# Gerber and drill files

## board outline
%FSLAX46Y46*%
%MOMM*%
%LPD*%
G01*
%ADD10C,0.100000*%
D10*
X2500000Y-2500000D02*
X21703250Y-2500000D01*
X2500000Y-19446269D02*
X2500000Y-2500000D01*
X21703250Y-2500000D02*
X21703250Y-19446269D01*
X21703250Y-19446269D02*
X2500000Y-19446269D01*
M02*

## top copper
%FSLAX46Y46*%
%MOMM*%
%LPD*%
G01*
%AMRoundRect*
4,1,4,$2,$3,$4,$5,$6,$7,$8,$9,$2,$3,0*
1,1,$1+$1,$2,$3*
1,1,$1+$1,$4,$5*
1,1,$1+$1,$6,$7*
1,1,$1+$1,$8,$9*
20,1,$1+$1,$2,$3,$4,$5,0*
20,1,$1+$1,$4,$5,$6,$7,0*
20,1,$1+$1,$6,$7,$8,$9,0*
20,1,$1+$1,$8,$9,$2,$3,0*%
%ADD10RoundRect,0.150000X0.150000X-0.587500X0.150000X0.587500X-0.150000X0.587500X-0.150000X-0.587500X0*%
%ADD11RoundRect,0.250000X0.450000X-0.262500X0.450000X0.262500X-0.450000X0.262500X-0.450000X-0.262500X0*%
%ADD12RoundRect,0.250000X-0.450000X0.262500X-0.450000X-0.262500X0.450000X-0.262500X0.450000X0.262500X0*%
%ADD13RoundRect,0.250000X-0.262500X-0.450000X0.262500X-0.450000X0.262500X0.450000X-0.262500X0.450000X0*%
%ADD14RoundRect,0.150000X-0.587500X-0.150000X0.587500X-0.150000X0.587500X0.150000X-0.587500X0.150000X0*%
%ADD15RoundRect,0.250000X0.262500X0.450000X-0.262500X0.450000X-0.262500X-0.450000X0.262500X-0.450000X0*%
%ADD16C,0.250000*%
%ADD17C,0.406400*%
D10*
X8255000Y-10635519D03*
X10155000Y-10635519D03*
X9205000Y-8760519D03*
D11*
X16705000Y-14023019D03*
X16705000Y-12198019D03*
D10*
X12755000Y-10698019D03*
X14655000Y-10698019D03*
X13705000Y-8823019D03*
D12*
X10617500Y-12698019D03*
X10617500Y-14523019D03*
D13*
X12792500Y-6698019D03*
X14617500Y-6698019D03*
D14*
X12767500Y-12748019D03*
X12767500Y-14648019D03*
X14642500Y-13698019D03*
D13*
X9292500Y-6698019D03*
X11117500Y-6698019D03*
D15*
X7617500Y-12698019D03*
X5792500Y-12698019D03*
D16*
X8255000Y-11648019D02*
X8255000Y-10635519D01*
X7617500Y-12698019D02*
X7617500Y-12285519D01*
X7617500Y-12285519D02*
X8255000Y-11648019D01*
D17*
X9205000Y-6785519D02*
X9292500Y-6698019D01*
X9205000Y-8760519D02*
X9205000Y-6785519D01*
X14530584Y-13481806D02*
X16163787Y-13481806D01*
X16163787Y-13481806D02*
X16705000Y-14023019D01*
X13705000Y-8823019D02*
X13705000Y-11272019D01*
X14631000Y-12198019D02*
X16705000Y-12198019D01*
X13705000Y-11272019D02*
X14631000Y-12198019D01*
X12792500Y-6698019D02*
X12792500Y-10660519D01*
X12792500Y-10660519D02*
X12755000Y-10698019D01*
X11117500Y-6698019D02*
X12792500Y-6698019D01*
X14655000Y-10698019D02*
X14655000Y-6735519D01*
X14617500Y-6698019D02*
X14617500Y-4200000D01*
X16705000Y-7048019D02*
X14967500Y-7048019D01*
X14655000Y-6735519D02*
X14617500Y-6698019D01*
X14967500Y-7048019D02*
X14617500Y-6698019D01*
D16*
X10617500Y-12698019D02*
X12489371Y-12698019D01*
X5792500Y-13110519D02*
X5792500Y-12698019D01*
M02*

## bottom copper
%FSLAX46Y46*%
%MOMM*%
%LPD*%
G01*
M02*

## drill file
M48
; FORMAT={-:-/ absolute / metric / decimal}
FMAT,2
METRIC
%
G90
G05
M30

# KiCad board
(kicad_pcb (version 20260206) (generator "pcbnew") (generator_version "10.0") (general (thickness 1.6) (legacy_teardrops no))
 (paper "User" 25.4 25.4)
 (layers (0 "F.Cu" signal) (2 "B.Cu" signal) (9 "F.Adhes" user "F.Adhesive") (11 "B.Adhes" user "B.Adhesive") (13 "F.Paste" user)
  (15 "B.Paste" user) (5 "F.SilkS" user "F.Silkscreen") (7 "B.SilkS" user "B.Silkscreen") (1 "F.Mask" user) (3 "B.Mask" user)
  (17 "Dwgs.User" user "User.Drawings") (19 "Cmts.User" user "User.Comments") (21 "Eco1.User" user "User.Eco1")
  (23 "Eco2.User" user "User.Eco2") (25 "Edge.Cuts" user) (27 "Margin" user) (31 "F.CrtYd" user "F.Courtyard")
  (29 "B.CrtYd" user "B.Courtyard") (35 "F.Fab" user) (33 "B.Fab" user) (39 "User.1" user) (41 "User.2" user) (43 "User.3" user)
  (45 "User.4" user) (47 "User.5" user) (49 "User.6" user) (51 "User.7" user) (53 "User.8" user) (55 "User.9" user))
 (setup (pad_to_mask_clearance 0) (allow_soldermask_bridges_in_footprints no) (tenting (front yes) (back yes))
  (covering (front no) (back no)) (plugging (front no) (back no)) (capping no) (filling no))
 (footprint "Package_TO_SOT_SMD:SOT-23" (layer "F.Cu") (at 9.205 9.698019 90)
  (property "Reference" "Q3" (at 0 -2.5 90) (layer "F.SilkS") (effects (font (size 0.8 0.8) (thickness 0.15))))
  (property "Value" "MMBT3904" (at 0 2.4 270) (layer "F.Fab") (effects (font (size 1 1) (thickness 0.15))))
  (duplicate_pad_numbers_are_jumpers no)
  (pad "1" smd roundrect (at -0.9375 -0.95 90) (size 1.475 0.6) (layers "F.Cu" "F.Mask" "F.Paste") (roundrect_rratio 0.25)
   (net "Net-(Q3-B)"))
  (pad "2" smd roundrect (at -0.9375 0.95 90) (size 1.475 0.6) (layers "F.Cu" "F.Mask" "F.Paste") (roundrect_rratio 0.25) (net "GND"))
  (pad "3" smd roundrect (at 0.9375 0 90) (size 1.475 0.6) (layers "F.Cu" "F.Mask" "F.Paste") (roundrect_rratio 0.25) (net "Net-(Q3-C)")))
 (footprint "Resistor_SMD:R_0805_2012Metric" (layer "F.Cu") (at 16.705 13.110519 90)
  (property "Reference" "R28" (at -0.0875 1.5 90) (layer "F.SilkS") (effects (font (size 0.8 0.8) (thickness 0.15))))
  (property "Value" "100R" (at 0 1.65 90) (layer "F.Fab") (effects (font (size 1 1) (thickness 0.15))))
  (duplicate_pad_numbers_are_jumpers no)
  (pad "1" smd roundrect (at -0.9125 0 90) (size 1.025 1.4) (layers "F.Cu" "F.Mask" "F.Paste") (roundrect_rratio 0.243902439)
   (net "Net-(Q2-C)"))
  (pad "2" smd roundrect (at 0.9125 0 90) (size 1.025 1.4) (layers "F.Cu" "F.Mask" "F.Paste") (roundrect_rratio 0.243902439) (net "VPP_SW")))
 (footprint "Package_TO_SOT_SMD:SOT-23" (layer "F.Cu") (at 13.705 9.760519 90)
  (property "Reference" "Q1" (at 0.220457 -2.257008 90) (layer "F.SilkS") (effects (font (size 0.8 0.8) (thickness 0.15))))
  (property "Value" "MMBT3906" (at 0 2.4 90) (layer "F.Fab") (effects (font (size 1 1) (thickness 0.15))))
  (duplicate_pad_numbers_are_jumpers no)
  (pad "1" smd roundrect (at -0.9375 -0.95 90) (size 1.475 0.6) (layers "F.Cu" "F.Mask" "F.Paste") (roundrect_rratio 0.25)
   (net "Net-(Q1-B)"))
  (pad "2" smd roundrect (at -0.9375 0.95 90) (size 1.475 0.6) (layers "F.Cu" "F.Mask" "F.Paste") (roundrect_rratio 0.25) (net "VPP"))
  (pad "3" smd roundrect (at 0.9375 0 90) (size 1.475 0.6) (layers "F.Cu" "F.Mask" "F.Paste") (roundrect_rratio 0.25) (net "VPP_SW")))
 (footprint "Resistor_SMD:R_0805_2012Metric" (layer "F.Cu") (at 10.6175 13.610519 -90)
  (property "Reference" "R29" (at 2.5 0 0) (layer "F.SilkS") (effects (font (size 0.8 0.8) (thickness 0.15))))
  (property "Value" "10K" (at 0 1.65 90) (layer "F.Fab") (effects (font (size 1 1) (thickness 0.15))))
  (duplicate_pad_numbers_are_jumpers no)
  (pad "1" smd roundrect (at -0.9125 0 270) (size 1.025 1.4) (layers "F.Cu" "F.Mask" "F.Paste") (roundrect_rratio 0.243902439)
   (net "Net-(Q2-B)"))
  (pad "2" smd roundrect (at 0.9125 0 270) (size 1.025 1.4) (layers "F.Cu" "F.Mask" "F.Paste") (roundrect_rratio 0.243902439)
   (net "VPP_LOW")))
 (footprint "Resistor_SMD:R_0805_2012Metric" (layer "F.Cu") (at 13.705 6.698019)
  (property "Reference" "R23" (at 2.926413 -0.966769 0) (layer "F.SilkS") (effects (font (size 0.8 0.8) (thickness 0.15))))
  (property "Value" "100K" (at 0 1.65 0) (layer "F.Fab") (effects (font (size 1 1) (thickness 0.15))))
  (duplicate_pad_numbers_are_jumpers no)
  (pad "1" smd roundrect (at -0.9125 0) (size 1.025 1.4) (layers "F.Cu" "F.Mask" "F.Paste") (roundrect_rratio 0.243902439)
   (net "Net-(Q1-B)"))
  (pad "2" smd roundrect (at 0.9125 0) (size 1.025 1.4) (layers "F.Cu" "F.Mask" "F.Paste") (roundrect_rratio 0.243902439) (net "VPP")))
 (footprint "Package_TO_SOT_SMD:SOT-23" (layer "F.Cu") (at 13.705 13.698019)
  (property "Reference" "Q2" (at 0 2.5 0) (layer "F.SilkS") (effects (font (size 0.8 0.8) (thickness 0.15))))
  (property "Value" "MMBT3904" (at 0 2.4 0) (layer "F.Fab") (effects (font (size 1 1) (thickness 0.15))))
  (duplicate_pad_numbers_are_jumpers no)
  (pad "1" smd roundrect (at -0.9375 -0.95) (size 1.475 0.6) (layers "F.Cu" "F.Mask" "F.Paste") (roundrect_rratio 0.25) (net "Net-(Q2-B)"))
  (pad "2" smd roundrect (at -0.9375 0.95) (size 1.475 0.6) (layers "F.Cu" "F.Mask" "F.Paste") (roundrect_rratio 0.25) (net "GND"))
  (pad "3" smd roundrect (at 0.9375 0) (size 1.475 0.6) (layers "F.Cu" "F.Mask" "F.Paste") (roundrect_rratio 0.25) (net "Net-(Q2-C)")))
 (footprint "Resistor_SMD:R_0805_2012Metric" (layer "F.Cu") (at 10.205 6.698019)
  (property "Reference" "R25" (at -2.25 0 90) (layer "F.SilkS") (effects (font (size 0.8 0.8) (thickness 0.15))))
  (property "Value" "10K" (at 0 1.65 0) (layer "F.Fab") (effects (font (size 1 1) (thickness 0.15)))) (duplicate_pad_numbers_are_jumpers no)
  (pad "1" smd roundrect (at -0.9125 0) (size 1.025 1.4) (layers "F.Cu" "F.Mask" "F.Paste") (roundrect_rratio 0.243902439)
   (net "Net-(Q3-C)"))
  (pad "2" smd roundrect (at 0.9125 0) (size 1.025 1.4) (layers "F.Cu" "F.Mask" "F.Paste") (roundrect_rratio 0.243902439) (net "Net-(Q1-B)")))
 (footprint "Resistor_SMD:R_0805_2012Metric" (layer "F.Cu") (at 6.705 12.698019 180)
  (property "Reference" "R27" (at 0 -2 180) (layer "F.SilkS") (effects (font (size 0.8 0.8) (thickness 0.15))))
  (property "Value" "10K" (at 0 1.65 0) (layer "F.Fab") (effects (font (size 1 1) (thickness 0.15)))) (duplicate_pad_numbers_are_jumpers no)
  (pad "1" smd roundrect (at -0.9125 0 180) (size 1.025 1.4) (layers "F.Cu" "F.Mask" "F.Paste") (roundrect_rratio 0.243902439)
   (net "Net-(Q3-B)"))
  (pad "2" smd roundrect (at 0.9125 0 180) (size 1.025 1.4) (layers "F.Cu" "F.Mask" "F.Paste") (roundrect_rratio 0.243902439)
   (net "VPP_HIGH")))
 (gr_line (start 2.5 2.5) (end 21.70325 2.5) (stroke (width 0.1) (type default)) (layer "Edge.Cuts"))
 (gr_line (start 2.5 19.446269) (end 2.5 2.5) (stroke (width 0.1) (type default)) (layer "Edge.Cuts"))
 (gr_line (start 21.70325 2.5) (end 21.70325 19.446269) (stroke (width 0.1) (type default)) (layer "Edge.Cuts"))
 (gr_line (start 21.70325 19.446269) (end 2.5 19.446269) (stroke (width 0.1) (type default)) (layer "Edge.Cuts"))
 (segment (start 8.255 11.648019) (end 8.255 10.635519) (width 0.25) (layer "F.Cu") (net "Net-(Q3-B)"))
 (segment (start 7.6175 12.698019) (end 7.6175 12.285519) (width 0.25) (layer "F.Cu") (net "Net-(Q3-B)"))
 (segment (start 7.6175 12.285519) (end 8.255 11.648019) (width 0.25) (layer "F.Cu") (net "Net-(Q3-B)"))
 (segment (start 9.205 6.785519) (end 9.2925 6.698019) (width 0.4064) (layer "F.Cu") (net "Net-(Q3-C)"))
 (segment (start 9.205 8.760519) (end 9.205 6.785519) (width 0.4064) (layer "F.Cu") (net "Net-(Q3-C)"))
 (segment (start 14.530584 13.481806) (end 16.163787 13.481806) (width 0.4064) (layer "F.Cu") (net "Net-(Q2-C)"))
 (segment (start 16.163787 13.481806) (end 16.705 14.023019) (width 0.4064) (layer "F.Cu") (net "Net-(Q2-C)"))
 (segment (start 13.705 8.823019) (end 13.705 11.272019) (width 0.4064) (layer "F.Cu") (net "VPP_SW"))
 (segment (start 14.631 12.198019) (end 16.705 12.198019) (width 0.4064) (layer "F.Cu") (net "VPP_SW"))
 (segment (start 13.705 11.272019) (end 14.631 12.198019) (width 0.4064) (layer "F.Cu") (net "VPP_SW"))
 (segment (start 12.7925 6.698019) (end 12.7925 10.660519) (width 0.4064) (layer "F.Cu") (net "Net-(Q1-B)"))
 (segment (start 12.7925 10.660519) (end 12.755 10.698019) (width 0.4064) (layer "F.Cu") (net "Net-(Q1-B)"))
 (segment (start 11.1175 6.698019) (end 12.7925 6.698019) (width 0.4064) (layer "F.Cu") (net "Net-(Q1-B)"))
 (segment (start 14.655 10.698019) (end 14.655 6.735519) (width 0.4064) (layer "F.Cu") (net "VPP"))
 (segment (start 14.6175 6.698019) (end 14.6175 4.2) (width 0.4064) (layer "F.Cu") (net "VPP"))
 (segment (start 16.705 7.048019) (end 14.9675 7.048019) (width 0.4064) (layer "F.Cu") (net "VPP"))
 (segment (start 14.655 6.735519) (end 14.6175 6.698019) (width 0.4064) (layer "F.Cu") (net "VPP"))
 (segment (start 14.9675 7.048019) (end 14.6175 6.698019) (width 0.4064) (layer "F.Cu") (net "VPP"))
 (segment (start 10.6175 12.698019) (end 12.489371 12.698019) (width 0.25) (layer "F.Cu") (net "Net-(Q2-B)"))
 (segment (start 5.7925 13.110519) (end 5.7925 12.698019) (width 0.25) (layer "F.Cu") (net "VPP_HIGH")))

